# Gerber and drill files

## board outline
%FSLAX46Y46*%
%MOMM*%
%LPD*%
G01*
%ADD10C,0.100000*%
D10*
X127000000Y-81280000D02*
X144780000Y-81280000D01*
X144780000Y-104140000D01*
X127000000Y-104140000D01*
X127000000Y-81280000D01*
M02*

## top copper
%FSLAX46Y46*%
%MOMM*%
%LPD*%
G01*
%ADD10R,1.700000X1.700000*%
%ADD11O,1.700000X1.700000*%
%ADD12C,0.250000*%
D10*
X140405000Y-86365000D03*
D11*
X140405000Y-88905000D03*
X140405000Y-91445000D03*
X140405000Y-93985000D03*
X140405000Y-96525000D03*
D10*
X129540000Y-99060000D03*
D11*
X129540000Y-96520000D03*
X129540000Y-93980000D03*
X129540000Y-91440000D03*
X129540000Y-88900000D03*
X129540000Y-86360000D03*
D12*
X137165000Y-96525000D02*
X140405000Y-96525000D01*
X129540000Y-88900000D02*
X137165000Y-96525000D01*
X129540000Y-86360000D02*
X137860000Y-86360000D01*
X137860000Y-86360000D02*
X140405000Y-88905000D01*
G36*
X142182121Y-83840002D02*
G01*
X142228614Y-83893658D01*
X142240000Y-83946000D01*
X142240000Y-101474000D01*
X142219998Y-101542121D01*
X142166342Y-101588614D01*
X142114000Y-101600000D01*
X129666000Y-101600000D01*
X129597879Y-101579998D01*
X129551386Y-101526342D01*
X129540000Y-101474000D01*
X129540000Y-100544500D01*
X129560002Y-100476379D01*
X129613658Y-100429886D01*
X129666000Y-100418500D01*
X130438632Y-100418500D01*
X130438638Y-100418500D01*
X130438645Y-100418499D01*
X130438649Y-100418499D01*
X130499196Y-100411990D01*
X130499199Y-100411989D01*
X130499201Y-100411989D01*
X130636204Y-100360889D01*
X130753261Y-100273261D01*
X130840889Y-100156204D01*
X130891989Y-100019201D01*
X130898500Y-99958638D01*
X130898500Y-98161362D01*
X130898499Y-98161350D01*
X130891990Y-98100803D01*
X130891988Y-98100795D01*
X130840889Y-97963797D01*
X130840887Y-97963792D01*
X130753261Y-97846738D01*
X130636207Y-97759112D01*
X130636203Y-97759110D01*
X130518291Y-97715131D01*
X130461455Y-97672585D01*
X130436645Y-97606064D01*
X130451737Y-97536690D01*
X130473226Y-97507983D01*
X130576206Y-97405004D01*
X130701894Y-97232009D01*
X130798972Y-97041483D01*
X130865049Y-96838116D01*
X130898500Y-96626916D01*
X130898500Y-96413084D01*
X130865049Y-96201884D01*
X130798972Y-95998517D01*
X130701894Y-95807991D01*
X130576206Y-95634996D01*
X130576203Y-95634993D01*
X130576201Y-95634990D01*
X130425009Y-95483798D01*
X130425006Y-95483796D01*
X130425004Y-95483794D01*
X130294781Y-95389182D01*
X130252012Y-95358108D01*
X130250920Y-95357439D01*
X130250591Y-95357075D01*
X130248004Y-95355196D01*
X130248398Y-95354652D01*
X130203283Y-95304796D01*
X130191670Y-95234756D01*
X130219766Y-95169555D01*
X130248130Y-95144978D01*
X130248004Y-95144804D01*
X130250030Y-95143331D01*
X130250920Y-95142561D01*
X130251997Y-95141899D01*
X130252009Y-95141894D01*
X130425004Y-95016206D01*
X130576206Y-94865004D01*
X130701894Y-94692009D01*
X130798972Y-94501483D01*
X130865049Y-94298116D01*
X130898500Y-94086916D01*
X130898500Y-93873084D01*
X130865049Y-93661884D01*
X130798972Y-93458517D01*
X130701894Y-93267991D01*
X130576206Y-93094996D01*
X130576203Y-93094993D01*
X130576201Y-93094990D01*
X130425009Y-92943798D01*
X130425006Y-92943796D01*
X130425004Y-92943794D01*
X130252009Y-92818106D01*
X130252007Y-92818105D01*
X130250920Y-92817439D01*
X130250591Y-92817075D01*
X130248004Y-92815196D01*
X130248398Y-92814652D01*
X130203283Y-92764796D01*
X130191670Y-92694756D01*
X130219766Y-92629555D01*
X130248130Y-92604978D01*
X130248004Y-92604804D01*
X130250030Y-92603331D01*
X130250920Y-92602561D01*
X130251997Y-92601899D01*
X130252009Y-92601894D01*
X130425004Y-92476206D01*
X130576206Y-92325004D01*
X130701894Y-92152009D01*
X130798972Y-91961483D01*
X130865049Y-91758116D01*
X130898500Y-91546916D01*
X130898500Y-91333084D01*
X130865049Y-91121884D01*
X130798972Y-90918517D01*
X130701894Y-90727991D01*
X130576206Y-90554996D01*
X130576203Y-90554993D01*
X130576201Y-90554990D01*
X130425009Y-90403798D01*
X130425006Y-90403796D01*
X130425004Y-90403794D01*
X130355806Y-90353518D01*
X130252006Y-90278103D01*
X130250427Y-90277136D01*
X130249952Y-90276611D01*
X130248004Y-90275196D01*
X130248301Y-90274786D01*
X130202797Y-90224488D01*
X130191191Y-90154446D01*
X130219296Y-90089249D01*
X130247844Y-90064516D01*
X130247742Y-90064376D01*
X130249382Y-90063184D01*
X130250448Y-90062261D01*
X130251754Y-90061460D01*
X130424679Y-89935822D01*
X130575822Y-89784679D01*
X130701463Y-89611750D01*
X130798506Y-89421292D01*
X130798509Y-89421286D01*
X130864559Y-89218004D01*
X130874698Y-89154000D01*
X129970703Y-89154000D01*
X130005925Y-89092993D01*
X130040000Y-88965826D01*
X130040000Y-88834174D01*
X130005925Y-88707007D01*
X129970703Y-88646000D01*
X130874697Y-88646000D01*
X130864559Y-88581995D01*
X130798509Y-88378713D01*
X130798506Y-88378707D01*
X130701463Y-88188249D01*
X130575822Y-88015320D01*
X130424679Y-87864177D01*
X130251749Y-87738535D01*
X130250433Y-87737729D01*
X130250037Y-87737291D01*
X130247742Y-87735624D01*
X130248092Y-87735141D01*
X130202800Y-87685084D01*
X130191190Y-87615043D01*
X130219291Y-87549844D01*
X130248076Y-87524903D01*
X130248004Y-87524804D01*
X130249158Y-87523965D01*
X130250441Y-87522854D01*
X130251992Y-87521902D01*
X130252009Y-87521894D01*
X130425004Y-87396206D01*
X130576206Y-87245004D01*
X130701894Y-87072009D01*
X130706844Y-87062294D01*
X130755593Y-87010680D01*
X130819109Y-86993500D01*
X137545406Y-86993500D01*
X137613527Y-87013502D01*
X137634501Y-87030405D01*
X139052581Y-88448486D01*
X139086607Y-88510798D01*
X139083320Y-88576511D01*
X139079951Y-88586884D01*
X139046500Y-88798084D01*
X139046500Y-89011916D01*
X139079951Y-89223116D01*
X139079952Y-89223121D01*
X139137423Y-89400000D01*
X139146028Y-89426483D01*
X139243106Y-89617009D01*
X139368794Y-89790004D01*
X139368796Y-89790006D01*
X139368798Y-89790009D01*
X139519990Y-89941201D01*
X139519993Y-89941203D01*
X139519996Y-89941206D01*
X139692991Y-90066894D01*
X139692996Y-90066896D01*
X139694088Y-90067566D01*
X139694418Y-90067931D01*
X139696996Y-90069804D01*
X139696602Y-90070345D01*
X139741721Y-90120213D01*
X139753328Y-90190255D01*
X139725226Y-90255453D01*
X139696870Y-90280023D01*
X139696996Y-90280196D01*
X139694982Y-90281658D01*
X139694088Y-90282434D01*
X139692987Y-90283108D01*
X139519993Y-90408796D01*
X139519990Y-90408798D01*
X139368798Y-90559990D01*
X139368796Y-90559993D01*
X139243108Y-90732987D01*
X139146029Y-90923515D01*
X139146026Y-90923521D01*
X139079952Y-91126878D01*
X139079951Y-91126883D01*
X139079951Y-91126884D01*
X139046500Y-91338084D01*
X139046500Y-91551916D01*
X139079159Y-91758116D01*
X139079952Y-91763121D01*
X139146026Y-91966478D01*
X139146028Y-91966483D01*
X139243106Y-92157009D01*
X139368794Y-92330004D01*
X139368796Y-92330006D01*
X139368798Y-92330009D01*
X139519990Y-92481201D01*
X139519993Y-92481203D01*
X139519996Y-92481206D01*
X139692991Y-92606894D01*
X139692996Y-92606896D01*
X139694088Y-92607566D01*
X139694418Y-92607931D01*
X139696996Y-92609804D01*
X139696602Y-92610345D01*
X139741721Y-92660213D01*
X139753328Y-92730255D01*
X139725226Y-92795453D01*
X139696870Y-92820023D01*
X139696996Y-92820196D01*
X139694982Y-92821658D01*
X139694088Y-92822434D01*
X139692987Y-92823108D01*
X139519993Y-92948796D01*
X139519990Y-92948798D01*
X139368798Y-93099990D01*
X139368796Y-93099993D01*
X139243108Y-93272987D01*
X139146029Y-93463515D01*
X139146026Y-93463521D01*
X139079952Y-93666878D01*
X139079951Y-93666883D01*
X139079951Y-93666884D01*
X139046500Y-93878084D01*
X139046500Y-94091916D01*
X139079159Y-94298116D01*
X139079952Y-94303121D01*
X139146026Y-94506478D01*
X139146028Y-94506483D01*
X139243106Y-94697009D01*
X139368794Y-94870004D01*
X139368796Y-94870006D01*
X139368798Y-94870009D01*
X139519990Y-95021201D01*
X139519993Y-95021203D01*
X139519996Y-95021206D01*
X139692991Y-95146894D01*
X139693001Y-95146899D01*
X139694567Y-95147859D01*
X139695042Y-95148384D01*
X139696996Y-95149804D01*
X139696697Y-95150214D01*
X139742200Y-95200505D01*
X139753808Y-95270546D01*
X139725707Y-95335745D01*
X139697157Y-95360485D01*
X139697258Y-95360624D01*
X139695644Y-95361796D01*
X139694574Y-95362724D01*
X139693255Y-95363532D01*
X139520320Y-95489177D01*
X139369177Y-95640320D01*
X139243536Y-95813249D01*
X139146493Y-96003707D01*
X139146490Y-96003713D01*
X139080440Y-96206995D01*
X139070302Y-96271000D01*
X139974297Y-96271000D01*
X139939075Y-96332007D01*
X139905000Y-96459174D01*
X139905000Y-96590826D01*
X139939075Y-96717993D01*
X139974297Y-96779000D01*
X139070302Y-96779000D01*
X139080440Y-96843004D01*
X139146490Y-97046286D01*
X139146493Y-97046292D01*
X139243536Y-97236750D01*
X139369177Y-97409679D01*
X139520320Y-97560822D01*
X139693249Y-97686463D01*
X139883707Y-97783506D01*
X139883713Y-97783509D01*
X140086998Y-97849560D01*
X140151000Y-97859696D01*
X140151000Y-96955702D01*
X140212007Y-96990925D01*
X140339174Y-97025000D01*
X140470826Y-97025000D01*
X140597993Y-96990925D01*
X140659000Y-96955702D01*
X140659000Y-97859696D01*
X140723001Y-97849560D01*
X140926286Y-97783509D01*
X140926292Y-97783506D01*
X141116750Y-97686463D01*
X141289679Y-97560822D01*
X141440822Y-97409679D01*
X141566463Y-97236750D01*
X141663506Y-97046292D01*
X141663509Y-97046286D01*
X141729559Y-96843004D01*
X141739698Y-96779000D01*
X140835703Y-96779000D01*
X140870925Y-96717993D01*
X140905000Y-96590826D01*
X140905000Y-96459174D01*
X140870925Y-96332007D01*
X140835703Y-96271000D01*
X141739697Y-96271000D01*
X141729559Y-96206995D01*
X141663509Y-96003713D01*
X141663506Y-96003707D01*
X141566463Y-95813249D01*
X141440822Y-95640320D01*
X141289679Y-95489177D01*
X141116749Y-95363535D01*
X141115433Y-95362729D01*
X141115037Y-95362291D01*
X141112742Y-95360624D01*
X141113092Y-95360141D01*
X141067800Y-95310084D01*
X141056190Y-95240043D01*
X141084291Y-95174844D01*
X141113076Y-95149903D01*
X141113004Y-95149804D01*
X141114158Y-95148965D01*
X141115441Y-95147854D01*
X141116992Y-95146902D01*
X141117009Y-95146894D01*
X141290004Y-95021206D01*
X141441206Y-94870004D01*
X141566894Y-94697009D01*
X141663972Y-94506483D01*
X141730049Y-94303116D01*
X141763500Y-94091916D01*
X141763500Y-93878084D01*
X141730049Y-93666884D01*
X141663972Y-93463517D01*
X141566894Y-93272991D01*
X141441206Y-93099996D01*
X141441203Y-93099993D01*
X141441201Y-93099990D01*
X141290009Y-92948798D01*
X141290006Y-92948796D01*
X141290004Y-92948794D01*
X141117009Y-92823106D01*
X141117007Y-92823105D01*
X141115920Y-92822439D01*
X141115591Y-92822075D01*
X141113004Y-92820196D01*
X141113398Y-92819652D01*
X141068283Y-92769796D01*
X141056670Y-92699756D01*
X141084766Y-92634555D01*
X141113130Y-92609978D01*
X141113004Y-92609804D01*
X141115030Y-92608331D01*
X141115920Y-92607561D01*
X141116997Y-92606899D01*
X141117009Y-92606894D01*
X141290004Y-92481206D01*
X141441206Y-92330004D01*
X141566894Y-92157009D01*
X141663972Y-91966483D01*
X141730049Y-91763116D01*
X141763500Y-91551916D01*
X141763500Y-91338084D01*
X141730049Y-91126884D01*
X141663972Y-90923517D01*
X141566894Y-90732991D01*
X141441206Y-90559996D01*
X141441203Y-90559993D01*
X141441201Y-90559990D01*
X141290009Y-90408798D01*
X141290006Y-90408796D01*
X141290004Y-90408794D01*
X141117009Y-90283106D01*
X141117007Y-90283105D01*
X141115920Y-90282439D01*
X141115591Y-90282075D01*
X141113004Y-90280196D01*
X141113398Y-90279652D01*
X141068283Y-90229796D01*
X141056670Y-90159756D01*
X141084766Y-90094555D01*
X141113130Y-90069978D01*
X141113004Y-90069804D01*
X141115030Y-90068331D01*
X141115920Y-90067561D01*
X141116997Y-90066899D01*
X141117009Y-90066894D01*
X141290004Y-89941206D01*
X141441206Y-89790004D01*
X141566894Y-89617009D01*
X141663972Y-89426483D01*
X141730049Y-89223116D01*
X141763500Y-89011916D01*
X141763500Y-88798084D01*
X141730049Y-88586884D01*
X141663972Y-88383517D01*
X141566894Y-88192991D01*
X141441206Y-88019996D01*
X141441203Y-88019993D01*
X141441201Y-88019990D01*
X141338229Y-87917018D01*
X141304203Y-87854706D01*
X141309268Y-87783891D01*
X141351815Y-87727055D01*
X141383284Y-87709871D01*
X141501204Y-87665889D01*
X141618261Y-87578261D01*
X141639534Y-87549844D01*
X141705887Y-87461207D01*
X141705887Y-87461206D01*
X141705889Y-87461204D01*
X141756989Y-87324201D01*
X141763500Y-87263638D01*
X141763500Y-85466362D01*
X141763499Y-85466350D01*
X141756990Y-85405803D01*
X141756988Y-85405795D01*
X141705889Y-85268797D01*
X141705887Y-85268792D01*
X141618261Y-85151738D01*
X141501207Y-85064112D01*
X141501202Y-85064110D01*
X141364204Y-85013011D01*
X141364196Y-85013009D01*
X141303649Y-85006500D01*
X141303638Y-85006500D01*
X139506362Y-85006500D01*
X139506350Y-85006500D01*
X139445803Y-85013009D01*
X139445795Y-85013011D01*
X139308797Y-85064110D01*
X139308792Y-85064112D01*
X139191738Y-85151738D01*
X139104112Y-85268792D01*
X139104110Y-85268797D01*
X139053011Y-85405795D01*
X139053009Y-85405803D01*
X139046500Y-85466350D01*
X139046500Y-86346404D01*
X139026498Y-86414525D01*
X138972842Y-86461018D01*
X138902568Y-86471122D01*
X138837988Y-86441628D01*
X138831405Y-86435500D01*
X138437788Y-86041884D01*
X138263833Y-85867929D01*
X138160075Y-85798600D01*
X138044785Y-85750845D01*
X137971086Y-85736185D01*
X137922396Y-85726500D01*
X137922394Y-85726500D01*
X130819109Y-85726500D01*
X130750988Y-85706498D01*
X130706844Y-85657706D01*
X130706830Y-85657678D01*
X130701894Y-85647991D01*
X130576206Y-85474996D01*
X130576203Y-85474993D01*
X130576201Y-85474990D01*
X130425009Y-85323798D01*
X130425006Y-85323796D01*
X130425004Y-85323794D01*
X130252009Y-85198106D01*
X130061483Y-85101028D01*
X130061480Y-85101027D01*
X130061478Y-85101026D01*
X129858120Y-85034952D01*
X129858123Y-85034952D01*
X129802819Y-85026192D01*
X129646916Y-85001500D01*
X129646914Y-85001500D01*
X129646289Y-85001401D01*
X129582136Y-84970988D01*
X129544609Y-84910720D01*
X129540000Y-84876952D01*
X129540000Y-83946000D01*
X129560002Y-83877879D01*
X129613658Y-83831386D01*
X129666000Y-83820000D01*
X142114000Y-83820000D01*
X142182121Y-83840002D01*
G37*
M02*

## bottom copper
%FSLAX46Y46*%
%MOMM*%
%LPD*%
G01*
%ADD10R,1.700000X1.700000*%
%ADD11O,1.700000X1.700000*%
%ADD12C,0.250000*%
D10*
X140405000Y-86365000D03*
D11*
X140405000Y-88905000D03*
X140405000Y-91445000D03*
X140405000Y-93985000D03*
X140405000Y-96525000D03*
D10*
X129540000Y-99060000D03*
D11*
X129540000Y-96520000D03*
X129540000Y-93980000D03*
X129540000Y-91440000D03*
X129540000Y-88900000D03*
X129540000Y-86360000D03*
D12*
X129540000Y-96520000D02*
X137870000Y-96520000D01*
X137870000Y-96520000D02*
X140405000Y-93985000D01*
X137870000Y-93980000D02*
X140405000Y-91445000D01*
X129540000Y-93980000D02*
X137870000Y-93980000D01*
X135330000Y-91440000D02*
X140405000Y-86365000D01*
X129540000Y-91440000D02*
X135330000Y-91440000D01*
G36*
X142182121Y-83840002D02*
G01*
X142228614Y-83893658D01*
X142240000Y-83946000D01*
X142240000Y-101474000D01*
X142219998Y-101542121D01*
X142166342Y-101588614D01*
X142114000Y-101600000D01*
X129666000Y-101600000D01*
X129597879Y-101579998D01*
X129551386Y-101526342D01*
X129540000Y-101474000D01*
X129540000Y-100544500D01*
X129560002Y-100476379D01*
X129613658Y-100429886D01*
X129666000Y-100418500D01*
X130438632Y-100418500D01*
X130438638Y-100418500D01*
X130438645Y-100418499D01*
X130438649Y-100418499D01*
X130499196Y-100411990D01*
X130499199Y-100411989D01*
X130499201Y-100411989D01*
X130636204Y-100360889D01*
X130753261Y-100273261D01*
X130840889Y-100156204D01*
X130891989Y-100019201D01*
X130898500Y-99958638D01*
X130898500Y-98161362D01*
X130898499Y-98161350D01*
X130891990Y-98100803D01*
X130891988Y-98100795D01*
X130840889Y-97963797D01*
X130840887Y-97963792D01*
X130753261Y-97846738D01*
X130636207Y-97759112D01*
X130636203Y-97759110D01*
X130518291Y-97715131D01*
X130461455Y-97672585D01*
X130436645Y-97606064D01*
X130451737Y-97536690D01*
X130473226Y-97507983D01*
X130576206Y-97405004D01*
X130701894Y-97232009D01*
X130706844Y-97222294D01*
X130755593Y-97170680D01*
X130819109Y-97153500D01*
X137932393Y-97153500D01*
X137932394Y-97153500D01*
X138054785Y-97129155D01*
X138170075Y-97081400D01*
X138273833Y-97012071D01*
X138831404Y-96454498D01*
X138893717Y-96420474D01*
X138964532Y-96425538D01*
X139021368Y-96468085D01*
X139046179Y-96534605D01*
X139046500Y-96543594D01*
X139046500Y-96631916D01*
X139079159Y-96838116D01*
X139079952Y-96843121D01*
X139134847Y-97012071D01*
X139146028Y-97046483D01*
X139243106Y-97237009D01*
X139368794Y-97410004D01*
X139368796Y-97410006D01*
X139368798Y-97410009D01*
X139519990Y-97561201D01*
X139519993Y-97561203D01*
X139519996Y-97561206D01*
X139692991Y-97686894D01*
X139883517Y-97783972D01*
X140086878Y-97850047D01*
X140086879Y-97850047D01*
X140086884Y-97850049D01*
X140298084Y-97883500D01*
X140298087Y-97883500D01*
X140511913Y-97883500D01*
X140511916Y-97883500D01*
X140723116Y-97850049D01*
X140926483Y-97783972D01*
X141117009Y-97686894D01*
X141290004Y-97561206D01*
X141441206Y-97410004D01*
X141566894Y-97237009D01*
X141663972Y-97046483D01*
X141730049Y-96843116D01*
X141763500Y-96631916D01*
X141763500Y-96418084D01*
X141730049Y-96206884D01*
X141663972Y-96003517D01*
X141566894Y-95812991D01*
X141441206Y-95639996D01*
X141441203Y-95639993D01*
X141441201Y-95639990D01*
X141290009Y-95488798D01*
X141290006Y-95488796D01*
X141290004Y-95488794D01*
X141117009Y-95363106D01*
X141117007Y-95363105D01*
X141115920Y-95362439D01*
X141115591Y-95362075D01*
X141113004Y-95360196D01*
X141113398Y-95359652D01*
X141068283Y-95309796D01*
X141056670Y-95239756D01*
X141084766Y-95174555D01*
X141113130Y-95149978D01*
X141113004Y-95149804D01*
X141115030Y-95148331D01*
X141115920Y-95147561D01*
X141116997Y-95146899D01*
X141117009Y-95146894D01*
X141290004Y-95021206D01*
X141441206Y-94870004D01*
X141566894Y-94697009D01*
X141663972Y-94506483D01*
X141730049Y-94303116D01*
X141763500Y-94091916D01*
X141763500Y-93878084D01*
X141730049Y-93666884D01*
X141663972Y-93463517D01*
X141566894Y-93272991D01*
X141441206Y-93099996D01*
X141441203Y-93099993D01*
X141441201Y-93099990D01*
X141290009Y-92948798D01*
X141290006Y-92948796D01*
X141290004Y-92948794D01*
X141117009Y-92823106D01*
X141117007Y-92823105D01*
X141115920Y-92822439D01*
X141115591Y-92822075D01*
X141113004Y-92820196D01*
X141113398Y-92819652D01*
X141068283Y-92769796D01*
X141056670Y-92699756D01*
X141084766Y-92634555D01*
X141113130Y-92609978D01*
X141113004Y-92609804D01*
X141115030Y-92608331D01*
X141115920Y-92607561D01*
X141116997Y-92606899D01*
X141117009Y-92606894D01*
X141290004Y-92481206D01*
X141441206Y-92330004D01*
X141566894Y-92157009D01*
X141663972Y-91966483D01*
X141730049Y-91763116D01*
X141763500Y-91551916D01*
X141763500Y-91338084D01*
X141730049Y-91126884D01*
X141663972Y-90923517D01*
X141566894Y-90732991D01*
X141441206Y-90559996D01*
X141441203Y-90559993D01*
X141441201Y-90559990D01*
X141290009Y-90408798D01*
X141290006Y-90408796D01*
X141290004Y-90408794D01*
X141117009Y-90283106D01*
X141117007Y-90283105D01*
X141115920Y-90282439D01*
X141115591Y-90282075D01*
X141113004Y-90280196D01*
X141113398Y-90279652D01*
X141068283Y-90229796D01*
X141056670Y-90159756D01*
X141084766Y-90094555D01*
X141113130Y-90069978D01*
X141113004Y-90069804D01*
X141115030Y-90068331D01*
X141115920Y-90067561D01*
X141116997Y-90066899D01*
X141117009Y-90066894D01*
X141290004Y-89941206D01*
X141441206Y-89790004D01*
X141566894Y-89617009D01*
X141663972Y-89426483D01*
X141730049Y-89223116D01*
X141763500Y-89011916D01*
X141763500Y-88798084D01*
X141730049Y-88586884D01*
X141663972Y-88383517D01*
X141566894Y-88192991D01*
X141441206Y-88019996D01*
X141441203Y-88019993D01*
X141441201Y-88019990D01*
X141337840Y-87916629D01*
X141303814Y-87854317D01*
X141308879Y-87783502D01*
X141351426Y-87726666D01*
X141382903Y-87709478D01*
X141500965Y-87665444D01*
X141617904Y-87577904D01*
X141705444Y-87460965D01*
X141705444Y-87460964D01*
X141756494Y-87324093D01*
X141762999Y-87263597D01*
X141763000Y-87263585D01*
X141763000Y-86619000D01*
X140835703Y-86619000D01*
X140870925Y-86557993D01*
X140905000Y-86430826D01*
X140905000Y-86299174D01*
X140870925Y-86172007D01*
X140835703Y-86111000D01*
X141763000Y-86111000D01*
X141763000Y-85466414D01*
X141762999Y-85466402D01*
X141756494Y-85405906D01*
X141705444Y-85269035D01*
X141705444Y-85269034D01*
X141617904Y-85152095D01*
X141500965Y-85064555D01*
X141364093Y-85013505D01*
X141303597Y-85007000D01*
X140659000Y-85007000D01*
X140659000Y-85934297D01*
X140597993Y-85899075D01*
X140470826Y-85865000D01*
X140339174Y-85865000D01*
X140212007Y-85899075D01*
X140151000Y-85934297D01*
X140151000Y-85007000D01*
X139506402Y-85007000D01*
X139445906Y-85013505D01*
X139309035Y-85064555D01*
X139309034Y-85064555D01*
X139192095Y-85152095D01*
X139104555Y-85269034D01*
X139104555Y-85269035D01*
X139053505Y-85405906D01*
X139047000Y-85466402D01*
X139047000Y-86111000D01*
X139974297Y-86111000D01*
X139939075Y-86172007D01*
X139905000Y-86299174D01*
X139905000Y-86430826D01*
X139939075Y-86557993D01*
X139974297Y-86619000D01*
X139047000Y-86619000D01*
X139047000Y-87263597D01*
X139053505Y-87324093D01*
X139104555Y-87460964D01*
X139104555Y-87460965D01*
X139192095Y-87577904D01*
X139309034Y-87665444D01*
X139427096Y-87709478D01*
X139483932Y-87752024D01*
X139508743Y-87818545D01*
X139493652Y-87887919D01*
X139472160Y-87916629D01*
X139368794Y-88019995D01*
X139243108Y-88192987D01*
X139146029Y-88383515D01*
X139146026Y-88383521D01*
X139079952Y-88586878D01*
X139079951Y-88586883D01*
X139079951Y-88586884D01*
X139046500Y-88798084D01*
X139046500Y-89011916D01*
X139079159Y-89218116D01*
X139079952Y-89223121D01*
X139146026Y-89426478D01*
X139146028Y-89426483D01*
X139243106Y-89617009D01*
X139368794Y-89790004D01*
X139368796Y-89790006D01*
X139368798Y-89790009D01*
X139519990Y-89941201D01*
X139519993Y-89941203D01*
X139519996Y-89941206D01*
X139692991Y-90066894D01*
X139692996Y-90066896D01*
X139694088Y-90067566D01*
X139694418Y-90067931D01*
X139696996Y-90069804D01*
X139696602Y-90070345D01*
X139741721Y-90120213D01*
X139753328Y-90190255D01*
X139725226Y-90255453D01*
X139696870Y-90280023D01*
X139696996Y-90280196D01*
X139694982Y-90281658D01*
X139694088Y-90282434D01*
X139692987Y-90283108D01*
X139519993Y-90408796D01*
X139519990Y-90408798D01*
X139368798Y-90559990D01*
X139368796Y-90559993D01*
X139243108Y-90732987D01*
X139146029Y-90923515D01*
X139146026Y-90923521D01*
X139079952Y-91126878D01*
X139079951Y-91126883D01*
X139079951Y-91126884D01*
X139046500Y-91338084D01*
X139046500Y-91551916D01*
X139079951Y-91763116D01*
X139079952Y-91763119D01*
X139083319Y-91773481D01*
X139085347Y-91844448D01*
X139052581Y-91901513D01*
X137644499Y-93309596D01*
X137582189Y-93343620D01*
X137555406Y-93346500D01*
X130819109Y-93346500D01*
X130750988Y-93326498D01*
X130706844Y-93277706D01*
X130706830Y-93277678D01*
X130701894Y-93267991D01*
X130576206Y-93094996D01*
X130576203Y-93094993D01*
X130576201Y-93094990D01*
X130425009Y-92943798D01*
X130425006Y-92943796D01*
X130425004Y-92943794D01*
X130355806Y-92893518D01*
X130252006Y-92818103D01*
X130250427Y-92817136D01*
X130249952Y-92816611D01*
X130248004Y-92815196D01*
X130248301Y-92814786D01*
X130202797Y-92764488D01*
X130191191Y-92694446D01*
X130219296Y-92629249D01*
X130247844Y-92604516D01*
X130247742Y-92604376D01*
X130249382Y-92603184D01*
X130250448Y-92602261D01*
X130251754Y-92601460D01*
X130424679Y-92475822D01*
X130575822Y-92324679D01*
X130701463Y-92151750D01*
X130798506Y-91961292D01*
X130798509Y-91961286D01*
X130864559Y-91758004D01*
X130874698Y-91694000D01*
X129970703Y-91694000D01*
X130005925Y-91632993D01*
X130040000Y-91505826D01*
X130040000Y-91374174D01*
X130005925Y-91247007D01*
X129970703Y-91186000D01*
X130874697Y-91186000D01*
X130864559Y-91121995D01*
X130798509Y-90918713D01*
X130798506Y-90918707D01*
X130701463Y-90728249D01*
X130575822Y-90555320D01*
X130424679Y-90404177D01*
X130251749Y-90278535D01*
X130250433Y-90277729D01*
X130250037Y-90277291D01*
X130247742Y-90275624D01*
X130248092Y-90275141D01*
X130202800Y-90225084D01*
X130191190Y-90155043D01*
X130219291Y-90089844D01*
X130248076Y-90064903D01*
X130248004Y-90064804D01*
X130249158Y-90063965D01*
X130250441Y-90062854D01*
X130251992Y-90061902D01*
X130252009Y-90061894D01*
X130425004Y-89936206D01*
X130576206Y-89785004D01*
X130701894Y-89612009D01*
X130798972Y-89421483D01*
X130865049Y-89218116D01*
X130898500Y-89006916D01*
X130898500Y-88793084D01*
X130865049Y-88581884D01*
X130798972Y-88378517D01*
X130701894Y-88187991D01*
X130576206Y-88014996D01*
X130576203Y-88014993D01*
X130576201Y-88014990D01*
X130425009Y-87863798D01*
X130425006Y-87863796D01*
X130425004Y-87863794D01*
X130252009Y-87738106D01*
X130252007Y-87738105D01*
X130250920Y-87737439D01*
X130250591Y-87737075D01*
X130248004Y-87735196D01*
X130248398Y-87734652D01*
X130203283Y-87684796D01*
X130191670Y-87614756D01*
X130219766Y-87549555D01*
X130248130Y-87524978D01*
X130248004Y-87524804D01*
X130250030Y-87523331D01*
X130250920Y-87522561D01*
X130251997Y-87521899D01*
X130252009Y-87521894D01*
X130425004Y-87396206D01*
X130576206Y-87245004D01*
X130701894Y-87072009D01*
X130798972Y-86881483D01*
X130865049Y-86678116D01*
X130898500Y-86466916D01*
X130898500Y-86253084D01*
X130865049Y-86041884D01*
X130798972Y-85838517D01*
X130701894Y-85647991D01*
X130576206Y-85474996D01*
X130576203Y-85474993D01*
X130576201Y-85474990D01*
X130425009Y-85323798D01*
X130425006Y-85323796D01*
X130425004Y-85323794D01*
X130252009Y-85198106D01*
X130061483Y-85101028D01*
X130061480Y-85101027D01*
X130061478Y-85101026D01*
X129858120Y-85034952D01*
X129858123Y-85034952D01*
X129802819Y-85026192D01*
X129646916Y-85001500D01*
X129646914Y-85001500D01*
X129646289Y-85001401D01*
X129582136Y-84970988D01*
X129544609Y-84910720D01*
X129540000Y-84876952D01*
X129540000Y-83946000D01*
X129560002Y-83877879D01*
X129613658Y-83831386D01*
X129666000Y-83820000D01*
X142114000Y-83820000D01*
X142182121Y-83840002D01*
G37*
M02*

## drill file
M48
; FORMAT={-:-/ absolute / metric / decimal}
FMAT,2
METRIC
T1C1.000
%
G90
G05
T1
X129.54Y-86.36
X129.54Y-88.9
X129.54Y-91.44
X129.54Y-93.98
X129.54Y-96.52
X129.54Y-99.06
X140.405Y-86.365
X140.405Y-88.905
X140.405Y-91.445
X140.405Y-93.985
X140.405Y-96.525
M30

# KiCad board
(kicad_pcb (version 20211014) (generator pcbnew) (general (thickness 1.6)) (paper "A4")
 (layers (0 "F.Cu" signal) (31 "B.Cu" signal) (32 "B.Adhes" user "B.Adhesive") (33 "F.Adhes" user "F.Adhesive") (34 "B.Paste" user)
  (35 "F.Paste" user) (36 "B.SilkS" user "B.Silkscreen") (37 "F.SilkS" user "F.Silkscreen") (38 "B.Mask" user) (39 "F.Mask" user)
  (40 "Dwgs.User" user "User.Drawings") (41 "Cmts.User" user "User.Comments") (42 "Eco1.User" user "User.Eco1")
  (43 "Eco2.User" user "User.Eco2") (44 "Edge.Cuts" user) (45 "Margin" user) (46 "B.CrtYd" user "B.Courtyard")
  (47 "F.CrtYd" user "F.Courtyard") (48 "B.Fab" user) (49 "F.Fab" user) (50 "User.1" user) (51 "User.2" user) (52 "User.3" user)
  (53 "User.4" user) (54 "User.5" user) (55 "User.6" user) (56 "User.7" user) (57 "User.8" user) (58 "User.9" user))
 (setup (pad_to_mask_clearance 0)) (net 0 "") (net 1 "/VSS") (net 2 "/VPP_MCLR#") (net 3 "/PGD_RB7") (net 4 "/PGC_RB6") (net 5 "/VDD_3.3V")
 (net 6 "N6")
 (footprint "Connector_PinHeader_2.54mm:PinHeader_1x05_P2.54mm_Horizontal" (layer "F.Cu") (at 140.405 86.365)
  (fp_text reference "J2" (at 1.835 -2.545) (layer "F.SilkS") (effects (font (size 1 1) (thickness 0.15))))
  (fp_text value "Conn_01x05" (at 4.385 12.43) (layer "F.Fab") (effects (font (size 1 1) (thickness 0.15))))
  (pad "1" thru_hole rect (at 0 0) (size 1.7 1.7) (drill 1) (layers *.Cu *.Mask) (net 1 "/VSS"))
  (pad "2" thru_hole oval (at 0 2.54) (size 1.7 1.7) (drill 1) (layers *.Cu *.Mask) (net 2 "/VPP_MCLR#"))
  (pad "3" thru_hole oval (at 0 5.08) (size 1.7 1.7) (drill 1) (layers *.Cu *.Mask) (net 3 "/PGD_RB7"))
  (pad "4" thru_hole oval (at 0 7.62) (size 1.7 1.7) (drill 1) (layers *.Cu *.Mask) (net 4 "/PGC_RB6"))
  (pad "5" thru_hole oval (at 0 10.16) (size 1.7 1.7) (drill 1) (layers *.Cu *.Mask) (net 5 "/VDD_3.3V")))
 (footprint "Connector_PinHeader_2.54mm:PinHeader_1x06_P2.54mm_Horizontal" (layer "F.Cu") (at 129.54 99.06 180)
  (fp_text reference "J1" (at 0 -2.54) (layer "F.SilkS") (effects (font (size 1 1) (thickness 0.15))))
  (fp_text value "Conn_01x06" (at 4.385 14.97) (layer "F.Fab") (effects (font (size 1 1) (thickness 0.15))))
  (pad "1" thru_hole rect (at 0 0 180) (size 1.7 1.7) (drill 1) (layers *.Cu *.Mask) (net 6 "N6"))
  (pad "2" thru_hole oval (at 0 2.54 180) (size 1.7 1.7) (drill 1) (layers *.Cu *.Mask) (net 4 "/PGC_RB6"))
  (pad "3" thru_hole oval (at 0 5.08 180) (size 1.7 1.7) (drill 1) (layers *.Cu *.Mask) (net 3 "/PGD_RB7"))
  (pad "4" thru_hole oval (at 0 7.62 180) (size 1.7 1.7) (drill 1) (layers *.Cu *.Mask) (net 1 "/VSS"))
  (pad "5" thru_hole oval (at 0 10.16 180) (size 1.7 1.7) (drill 1) (layers *.Cu *.Mask) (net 5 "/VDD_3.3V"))
  (pad "6" thru_hole oval (at 0 12.7 180) (size 1.7 1.7) (drill 1) (layers *.Cu *.Mask) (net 2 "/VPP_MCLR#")))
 (gr_rect (start 127 104.14) (end 144.78 81.28) (layer "Edge.Cuts") (width 0.1) (fill none))
 (segment (start 129.54 96.52) (end 137.87 96.52) (width 0.25) (layer "B.Cu") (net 4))
 (segment (start 137.87 96.52) (end 140.405 93.985) (width 0.25) (layer "B.Cu") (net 4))
 (segment (start 137.87 93.98) (end 140.405 91.445) (width 0.25) (layer "B.Cu") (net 3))
 (segment (start 129.54 93.98) (end 137.87 93.98) (width 0.25) (layer "B.Cu") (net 3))
 (segment (start 135.33 91.44) (end 140.405 86.365) (width 0.25) (layer "B.Cu") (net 1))
 (segment (start 129.54 91.44) (end 135.33 91.44) (width 0.25) (layer "B.Cu") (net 1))
 (segment (start 137.165 96.525) (end 140.405 96.525) (width 0.25) (layer "F.Cu") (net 5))
 (segment (start 129.54 88.9) (end 137.165 96.525) (width 0.25) (layer "F.Cu") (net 5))
 (segment (start 129.54 86.36) (end 137.86 86.36) (width 0.25) (layer "F.Cu") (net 2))
 (segment (start 137.86 86.36) (end 140.405 88.905) (width 0.25) (layer "F.Cu") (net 2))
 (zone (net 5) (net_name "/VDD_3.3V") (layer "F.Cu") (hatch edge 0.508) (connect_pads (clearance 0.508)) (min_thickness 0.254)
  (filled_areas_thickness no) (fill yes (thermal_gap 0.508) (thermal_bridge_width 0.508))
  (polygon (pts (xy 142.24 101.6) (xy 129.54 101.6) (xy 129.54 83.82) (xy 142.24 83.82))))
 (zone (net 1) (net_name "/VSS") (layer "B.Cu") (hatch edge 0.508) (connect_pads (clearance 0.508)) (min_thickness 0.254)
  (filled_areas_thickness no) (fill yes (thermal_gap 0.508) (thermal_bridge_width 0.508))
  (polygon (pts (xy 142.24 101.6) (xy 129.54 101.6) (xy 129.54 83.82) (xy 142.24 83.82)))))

